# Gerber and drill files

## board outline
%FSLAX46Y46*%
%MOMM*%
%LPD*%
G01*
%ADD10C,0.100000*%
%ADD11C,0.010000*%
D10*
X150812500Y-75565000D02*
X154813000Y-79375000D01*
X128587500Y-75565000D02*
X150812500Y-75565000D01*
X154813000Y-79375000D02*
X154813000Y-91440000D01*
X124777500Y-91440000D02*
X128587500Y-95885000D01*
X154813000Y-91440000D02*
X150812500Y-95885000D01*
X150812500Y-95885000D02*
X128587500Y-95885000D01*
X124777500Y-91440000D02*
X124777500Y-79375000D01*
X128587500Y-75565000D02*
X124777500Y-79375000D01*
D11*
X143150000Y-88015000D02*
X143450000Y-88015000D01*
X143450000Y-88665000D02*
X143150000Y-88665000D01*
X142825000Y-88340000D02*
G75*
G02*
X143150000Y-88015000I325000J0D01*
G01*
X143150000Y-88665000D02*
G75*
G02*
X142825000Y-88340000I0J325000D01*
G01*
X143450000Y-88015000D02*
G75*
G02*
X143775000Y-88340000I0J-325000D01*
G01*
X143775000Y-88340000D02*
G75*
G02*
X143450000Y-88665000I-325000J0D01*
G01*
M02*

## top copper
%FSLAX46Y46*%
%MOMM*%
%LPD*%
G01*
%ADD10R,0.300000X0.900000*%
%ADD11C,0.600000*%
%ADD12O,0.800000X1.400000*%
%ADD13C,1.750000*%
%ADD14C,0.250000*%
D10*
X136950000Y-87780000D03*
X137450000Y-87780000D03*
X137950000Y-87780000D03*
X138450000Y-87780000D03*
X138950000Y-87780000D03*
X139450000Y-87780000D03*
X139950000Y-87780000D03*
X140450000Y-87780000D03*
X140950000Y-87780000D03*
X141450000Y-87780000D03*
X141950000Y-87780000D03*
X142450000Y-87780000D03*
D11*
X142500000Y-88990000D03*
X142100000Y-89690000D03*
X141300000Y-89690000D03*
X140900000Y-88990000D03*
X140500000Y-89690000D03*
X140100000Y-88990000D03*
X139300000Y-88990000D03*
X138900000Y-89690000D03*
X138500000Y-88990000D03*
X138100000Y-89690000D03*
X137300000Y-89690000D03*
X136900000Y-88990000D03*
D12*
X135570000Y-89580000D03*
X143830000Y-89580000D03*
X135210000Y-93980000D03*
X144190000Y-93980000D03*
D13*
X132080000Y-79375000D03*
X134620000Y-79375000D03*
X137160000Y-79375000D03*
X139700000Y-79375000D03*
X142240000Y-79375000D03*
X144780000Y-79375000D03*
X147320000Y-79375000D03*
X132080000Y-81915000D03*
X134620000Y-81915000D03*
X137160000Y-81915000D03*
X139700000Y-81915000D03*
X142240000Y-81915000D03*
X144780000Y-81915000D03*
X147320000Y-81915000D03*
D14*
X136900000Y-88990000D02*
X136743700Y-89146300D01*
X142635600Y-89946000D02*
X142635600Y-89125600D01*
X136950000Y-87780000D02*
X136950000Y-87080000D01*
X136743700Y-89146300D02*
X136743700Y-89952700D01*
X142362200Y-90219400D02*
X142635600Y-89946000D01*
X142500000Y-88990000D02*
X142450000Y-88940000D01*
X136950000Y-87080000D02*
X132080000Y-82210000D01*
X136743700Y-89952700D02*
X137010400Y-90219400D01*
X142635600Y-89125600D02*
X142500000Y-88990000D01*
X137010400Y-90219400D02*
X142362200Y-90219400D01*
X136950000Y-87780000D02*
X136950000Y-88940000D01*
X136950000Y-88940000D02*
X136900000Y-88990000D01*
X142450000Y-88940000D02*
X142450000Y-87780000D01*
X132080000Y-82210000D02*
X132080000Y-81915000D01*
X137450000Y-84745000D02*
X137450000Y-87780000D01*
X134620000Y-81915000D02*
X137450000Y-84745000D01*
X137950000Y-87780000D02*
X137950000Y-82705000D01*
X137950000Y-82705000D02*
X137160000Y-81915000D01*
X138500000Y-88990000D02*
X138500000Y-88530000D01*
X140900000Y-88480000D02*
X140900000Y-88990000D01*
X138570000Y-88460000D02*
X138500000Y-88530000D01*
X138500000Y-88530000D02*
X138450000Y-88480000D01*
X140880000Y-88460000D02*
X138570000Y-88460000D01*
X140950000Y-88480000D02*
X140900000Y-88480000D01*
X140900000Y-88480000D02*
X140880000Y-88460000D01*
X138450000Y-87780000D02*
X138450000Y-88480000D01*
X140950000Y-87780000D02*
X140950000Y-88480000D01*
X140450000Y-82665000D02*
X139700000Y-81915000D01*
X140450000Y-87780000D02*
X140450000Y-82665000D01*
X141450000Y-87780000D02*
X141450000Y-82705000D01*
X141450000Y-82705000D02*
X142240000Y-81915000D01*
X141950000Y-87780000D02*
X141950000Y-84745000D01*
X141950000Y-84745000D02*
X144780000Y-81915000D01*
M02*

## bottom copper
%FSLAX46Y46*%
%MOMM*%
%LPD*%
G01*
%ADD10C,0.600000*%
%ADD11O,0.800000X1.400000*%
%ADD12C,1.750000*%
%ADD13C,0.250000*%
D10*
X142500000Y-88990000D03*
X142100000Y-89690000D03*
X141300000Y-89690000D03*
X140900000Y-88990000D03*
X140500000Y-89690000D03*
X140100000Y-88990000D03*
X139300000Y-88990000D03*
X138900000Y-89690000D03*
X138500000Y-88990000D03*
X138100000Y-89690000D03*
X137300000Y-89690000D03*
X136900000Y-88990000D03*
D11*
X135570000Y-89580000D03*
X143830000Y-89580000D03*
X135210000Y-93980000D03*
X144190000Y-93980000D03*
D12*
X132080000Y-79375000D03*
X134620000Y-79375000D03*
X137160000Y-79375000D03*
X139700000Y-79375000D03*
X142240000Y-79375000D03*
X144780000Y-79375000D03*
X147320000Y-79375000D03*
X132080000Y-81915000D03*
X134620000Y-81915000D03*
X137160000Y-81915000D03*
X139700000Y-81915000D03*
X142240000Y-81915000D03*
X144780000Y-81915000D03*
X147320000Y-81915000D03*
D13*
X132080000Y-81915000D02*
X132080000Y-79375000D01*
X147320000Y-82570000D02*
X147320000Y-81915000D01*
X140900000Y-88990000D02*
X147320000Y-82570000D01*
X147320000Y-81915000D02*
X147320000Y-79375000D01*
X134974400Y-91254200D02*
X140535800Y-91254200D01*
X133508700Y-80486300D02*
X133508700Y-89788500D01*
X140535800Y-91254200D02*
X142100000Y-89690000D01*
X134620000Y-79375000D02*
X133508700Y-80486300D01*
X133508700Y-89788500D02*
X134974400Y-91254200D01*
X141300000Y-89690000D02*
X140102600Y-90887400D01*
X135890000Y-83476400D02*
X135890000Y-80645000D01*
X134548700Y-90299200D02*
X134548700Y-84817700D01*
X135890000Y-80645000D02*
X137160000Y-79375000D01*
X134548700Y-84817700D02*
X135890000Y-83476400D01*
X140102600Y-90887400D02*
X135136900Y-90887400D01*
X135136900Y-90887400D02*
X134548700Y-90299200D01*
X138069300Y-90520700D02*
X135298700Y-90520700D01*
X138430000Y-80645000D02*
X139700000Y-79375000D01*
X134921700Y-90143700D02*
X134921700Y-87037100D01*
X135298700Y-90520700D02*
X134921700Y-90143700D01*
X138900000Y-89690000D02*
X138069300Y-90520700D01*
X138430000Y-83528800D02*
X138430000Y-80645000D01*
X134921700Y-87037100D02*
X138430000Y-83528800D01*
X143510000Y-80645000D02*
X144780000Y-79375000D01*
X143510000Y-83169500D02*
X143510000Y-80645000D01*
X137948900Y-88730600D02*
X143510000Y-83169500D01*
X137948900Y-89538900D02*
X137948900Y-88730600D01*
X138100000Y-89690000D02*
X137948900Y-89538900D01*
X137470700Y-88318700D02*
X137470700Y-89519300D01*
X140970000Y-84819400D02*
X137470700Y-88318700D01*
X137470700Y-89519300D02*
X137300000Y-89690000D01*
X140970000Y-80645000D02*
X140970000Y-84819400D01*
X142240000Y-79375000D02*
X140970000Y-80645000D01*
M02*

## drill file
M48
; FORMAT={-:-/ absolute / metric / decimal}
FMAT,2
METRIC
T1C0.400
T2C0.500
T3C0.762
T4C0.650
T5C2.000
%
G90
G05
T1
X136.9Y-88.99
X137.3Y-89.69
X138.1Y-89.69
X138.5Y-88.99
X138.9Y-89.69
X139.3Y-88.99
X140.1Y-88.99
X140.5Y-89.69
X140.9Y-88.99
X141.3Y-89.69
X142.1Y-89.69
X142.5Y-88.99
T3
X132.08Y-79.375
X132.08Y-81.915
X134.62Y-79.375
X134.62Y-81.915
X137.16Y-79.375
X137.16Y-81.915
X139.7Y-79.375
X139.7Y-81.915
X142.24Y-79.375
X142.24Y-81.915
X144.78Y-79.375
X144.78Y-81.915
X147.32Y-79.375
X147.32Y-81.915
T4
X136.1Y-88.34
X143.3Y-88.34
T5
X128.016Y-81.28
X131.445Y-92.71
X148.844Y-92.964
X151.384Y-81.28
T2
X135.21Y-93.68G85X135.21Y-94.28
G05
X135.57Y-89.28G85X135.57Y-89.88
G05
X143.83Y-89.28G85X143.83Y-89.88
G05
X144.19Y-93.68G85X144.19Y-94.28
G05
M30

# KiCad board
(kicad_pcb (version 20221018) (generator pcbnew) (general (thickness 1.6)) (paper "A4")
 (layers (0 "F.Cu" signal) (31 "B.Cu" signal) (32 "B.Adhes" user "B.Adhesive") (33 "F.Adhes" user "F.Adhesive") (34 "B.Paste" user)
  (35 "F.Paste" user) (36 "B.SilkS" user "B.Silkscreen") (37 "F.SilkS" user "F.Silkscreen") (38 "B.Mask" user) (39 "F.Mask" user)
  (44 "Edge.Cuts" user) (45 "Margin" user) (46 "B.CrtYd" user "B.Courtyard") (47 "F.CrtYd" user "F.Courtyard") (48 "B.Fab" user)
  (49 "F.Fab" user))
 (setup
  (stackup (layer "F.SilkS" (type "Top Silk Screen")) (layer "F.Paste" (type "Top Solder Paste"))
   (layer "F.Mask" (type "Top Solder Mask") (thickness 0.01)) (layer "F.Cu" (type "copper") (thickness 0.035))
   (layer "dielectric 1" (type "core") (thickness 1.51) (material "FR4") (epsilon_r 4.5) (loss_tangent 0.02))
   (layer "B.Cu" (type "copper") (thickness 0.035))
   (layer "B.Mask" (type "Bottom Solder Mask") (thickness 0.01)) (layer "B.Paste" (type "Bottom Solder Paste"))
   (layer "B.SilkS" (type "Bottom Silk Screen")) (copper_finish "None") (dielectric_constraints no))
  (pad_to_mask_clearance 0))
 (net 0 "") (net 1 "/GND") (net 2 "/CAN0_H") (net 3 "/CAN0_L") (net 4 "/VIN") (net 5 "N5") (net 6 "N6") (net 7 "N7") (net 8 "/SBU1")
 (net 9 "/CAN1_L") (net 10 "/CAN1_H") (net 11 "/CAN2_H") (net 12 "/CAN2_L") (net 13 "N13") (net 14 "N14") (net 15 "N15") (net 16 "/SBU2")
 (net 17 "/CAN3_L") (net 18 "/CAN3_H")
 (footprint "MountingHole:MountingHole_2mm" (layer "F.Cu") (at 128.016 81.28)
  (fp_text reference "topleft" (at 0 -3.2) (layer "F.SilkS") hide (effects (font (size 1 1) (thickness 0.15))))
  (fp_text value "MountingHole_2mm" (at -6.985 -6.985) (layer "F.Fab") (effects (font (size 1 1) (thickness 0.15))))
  (pad "" np_thru_hole circle (at 0 0) (size 2 2) (drill 2) (layers "*.Cu" "*.Mask")))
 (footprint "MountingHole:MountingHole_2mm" (layer "F.Cu") (at 148.844 92.964)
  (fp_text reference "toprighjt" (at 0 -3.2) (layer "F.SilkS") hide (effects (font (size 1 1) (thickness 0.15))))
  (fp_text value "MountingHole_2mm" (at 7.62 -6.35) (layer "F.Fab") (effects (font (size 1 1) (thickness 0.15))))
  (pad "" np_thru_hole circle (at 0 0) (size 2 2) (drill 2) (layers "F&B.Cu" "*.Mask")))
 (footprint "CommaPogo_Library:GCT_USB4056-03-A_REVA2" (layer "F.Cu") (at 139.7 93.98)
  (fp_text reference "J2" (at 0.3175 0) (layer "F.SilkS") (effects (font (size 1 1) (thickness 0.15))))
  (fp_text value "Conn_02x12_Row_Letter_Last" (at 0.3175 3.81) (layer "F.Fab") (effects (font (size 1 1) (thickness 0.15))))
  (fp_line (start 3.45 -5.965) (end 3.75 -5.965) (stroke (width 0.01) (type solid)) (layer "Edge.Cuts"))
  (fp_line (start 3.75 -5.315) (end 3.45 -5.315) (stroke (width 0.01) (type solid)) (layer "Edge.Cuts"))
  (fp_arc (start 3.125 -5.64) (mid 3.22019 -5.86981) (end 3.45 -5.965) (stroke (width 0.01) (type solid)) (layer "Edge.Cuts"))
  (fp_arc (start 3.45 -5.315) (mid 3.22019 -5.41019) (end 3.125 -5.64) (stroke (width 0.01) (type solid)) (layer "Edge.Cuts"))
  (fp_arc (start 3.75 -5.965) (mid 3.97981 -5.86981) (end 4.075 -5.64) (stroke (width 0.01) (type solid)) (layer "Edge.Cuts"))
  (fp_arc (start 4.075 -5.64) (mid 3.97981 -5.41019) (end 3.75 -5.315) (stroke (width 0.01) (type solid)) (layer "Edge.Cuts"))
  (pad "" np_thru_hole circle (at -3.6 -5.64) (size 0.65 0.65) (drill 0.65) (layers "*.Cu" "*.Mask"))
  (pad "" np_thru_hole circle (at 3.6 -5.64) (size 0.65 0.65) (drill 0.65) (layers "*.Cu" "*.Mask"))
  (pad "A1" smd rect (at -2.75 -6.2) (size 0.3 0.9) (layers "F.Cu" "F.Paste" "F.Mask") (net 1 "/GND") (solder_mask_margin 0.102))
  (pad "A2" smd rect (at -2.25 -6.2) (size 0.3 0.9) (layers "F.Cu" "F.Paste" "F.Mask") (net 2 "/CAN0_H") (solder_mask_margin 0.102))
  (pad "A3" smd rect (at -1.75 -6.2) (size 0.3 0.9) (layers "F.Cu" "F.Paste" "F.Mask") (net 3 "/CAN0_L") (solder_mask_margin 0.102))
  (pad "A4" smd rect (at -1.25 -6.2) (size 0.3 0.9) (layers "F.Cu" "F.Paste" "F.Mask") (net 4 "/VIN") (solder_mask_margin 0.102))
  (pad "A5" smd rect (at -0.75 -6.2) (size 0.3 0.9) (layers "F.Cu" "F.Paste" "F.Mask") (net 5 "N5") (solder_mask_margin 0.102))
  (pad "A6" smd rect (at -0.25 -6.2) (size 0.3 0.9) (layers "F.Cu" "F.Paste" "F.Mask") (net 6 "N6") (solder_mask_margin 0.102))
  (pad "A7" smd rect (at 0.25 -6.2) (size 0.3 0.9) (layers "F.Cu" "F.Paste" "F.Mask") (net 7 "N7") (solder_mask_margin 0.102))
  (pad "A8" smd rect (at 0.75 -6.2) (size 0.3 0.9) (layers "F.Cu" "F.Paste" "F.Mask") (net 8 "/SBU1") (solder_mask_margin 0.102))
  (pad "A9" smd rect (at 1.25 -6.2) (size 0.3 0.9) (layers "F.Cu" "F.Paste" "F.Mask") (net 4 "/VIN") (solder_mask_margin 0.102))
  (pad "A10" smd rect (at 1.75 -6.2) (size 0.3 0.9) (layers "F.Cu" "F.Paste" "F.Mask") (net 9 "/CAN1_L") (solder_mask_margin 0.102))
  (pad "A11" smd rect (at 2.25 -6.2) (size 0.3 0.9) (layers "F.Cu" "F.Paste" "F.Mask") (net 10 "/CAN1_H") (solder_mask_margin 0.102))
  (pad "A12" smd rect (at 2.75 -6.2) (size 0.3 0.9) (layers "F.Cu" "F.Paste" "F.Mask") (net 1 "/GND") (solder_mask_margin 0.102))
  (pad "B1" thru_hole circle (at 2.8 -4.99) (size 0.6 0.6) (drill 0.4) (layers "*.Cu" "*.Mask") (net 1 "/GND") (solder_mask_margin 0.102))
  (pad "B2" thru_hole circle (at 2.4 -4.29) (size 0.6 0.6) (drill 0.4) (layers "*.Cu" "*.Mask") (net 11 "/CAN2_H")
   (solder_mask_margin 0.102))
  (pad "B3" thru_hole circle (at 1.6 -4.29) (size 0.6 0.6) (drill 0.4) (layers "*.Cu" "*.Mask") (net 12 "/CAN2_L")
   (solder_mask_margin 0.102))
  (pad "B4" thru_hole circle (at 1.2 -4.99) (size 0.6 0.6) (drill 0.4) (layers "*.Cu" "*.Mask") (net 4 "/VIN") (solder_mask_margin 0.102))
  (pad "B5" thru_hole circle (at 0.8 -4.29) (size 0.6 0.6) (drill 0.4) (layers "*.Cu" "*.Mask") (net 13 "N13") (solder_mask_margin 0.102))
  (pad "B6" thru_hole circle (at 0.4 -4.99) (size 0.6 0.6) (drill 0.4) (layers "*.Cu" "*.Mask") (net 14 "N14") (solder_mask_margin 0.102))
  (pad "B7" thru_hole circle (at -0.4 -4.99) (size 0.6 0.6) (drill 0.4) (layers "*.Cu" "*.Mask") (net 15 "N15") (solder_mask_margin 0.102))
  (pad "B8" thru_hole circle (at -0.8 -4.29) (size 0.6 0.6) (drill 0.4) (layers "*.Cu" "*.Mask") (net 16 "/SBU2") (solder_mask_margin 0.102))
  (pad "B9" thru_hole circle (at -1.2 -4.99) (size 0.6 0.6) (drill 0.4) (layers "*.Cu" "*.Mask") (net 4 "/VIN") (solder_mask_margin 0.102))
  (pad "B10" thru_hole circle (at -1.6 -4.29) (size 0.6 0.6) (drill 0.4) (layers "*.Cu" "*.Mask") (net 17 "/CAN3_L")
   (solder_mask_margin 0.102))
  (pad "B11" thru_hole circle (at -2.4 -4.29) (size 0.6 0.6) (drill 0.4) (layers "*.Cu" "*.Mask") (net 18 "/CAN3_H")
   (solder_mask_margin 0.102))
  (pad "B12" thru_hole circle (at -2.8 -4.99) (size 0.6 0.6) (drill 0.4) (layers "*.Cu" "*.Mask") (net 1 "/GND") (solder_mask_margin 0.102))
  (pad "S1" thru_hole oval (at -4.13 -4.4) (size 0.8 1.4) (drill oval 0.5 1.1) (layers "*.Cu" "*.Mask") (solder_mask_margin 0.102))
  (pad "S2" thru_hole oval (at 4.13 -4.4) (size 0.8 1.4) (drill oval 0.5 1.1) (layers "*.Cu" "*.Mask") (solder_mask_margin 0.102))
  (pad "S3" thru_hole oval (at -4.49 0) (size 0.8 1.4) (drill oval 0.5 1.1) (layers "*.Cu" "*.Mask") (solder_mask_margin 0.102))
  (pad "S4" thru_hole oval (at 4.49 0) (size 0.8 1.4) (drill oval 0.5 1.1) (layers "*.Cu" "*.Mask") (solder_mask_margin 0.102)))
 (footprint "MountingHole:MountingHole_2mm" (layer "F.Cu") (at 151.384 81.28)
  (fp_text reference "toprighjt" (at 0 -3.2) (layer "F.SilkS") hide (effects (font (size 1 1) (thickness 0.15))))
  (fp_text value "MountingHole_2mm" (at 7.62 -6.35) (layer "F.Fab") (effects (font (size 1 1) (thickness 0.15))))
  (pad "" np_thru_hole circle (at 0 0) (size 2 2) (drill 2) (layers "*.Cu" "*.Mask")))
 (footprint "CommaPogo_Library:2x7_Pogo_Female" (layer "F.Cu") (at 139.7 83.82)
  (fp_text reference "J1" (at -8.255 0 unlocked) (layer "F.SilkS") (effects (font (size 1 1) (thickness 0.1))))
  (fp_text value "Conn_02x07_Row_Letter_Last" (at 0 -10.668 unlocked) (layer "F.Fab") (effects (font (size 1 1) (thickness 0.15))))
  (pad "1" thru_hole circle (at -7.62 -4.445) (size 1.75 1.75) (drill 0.762) (layers "*.Cu" "*.Mask") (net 1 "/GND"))
  (pad "2" thru_hole circle (at -5.08 -4.445) (size 1.75 1.75) (drill 0.762) (layers "*.Cu" "*.Mask") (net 11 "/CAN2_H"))
  (pad "3" thru_hole circle (at -2.54 -4.445) (size 1.75 1.75) (drill 0.762) (layers "*.Cu" "*.Mask") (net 12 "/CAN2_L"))
  (pad "4" thru_hole circle (at 0 -4.445) (size 1.75 1.75) (drill 0.762) (layers "*.Cu" "*.Mask") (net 16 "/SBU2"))
  (pad "5" thru_hole circle (at 2.54 -4.445) (size 1.75 1.75) (drill 0.762) (layers "*.Cu" "*.Mask") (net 18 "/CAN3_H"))
  (pad "6" thru_hole circle (at 5.08 -4.445) (size 1.75 1.75) (drill 0.762) (layers "*.Cu" "*.Mask") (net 17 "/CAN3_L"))
  (pad "7" thru_hole circle (at 7.62 -4.445) (size 1.75 1.75) (drill 0.762) (layers "*.Cu" "*.Mask") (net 4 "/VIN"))
  (pad "8" thru_hole circle (at -7.62 -1.905) (size 1.75 1.75) (drill 0.762) (layers "*.Cu" "*.Mask") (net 1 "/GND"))
  (pad "9" thru_hole circle (at -5.08 -1.905) (size 1.75 1.75) (drill 0.762) (layers "*.Cu" "*.Mask") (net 2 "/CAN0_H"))
  (pad "10" thru_hole circle (at -2.54 -1.905) (size 1.75 1.75) (drill 0.762) (layers "*.Cu" "*.Mask") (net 3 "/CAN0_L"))
  (pad "11" thru_hole circle (at 0 -1.905) (size 1.75 1.75) (drill 0.762) (layers "*.Cu" "*.Mask") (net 8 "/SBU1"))
  (pad "12" thru_hole circle (at 2.54 -1.905) (size 1.75 1.75) (drill 0.762) (layers "*.Cu" "*.Mask") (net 9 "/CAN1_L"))
  (pad "13" thru_hole circle (at 5.08 -1.905) (size 1.75 1.75) (drill 0.762) (layers "*.Cu" "*.Mask") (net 10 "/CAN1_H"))
  (pad "14" thru_hole circle (at 7.62 -1.905) (size 1.75 1.75) (drill 0.762) (layers "*.Cu" "*.Mask") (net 4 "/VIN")))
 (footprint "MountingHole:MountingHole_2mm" (layer "F.Cu") (at 131.445 92.71)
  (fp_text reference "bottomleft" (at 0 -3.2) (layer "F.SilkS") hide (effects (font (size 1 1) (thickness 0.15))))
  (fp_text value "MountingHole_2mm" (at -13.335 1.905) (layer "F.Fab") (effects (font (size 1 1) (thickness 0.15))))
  (pad "" np_thru_hole circle (at 0 0) (size 2 2) (drill 2) (layers "F&B.Cu" "*.Mask")))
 (gr_line (start 150.8125 75.565) (end 154.813 79.375) (stroke (width 0.1) (type default)) (layer "Edge.Cuts"))
 (gr_line (start 128.5875 75.565) (end 150.8125 75.565) (stroke (width 0.1) (type default)) (layer "Edge.Cuts"))
 (gr_line (start 154.813 79.375) (end 154.813 91.44) (stroke (width 0.1) (type default)) (layer "Edge.Cuts"))
 (gr_line (start 124.7775 91.44) (end 128.5875 95.885) (stroke (width 0.1) (type default)) (layer "Edge.Cuts"))
 (gr_line (start 154.813 91.44) (end 150.8125 95.885) (stroke (width 0.1) (type default)) (layer "Edge.Cuts"))
 (gr_line (start 150.8125 95.885) (end 128.5875 95.885) (stroke (width 0.1) (type default)) (layer "Edge.Cuts"))
 (gr_line (start 124.7775 91.44) (end 124.7775 79.375) (stroke (width 0.1) (type default)) (layer "Edge.Cuts"))
 (gr_line (start 128.5875 75.565) (end 124.7775 79.375) (stroke (width 0.1) (type default)) (layer "Edge.Cuts"))
 (segment (start 136.9 88.99) (end 136.7437 89.1463) (width 0.25) (layer "F.Cu") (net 1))
 (segment (start 142.6356 89.946) (end 142.6356 89.1256) (width 0.25) (layer "F.Cu") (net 1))
 (segment (start 136.95 87.78) (end 136.95 87.08) (width 0.25) (layer "F.Cu") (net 1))
 (segment (start 136.7437 89.1463) (end 136.7437 89.9527) (width 0.25) (layer "F.Cu") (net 1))
 (segment (start 142.3622 90.2194) (end 142.6356 89.946) (width 0.25) (layer "F.Cu") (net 1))
 (segment (start 142.5 88.99) (end 142.45 88.94) (width 0.25) (layer "F.Cu") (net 1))
 (segment (start 136.95 87.08) (end 132.08 82.21) (width 0.25) (layer "F.Cu") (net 1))
 (segment (start 136.7437 89.9527) (end 137.0104 90.2194) (width 0.25) (layer "F.Cu") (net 1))
 (segment (start 142.6356 89.1256) (end 142.5 88.99) (width 0.25) (layer "F.Cu") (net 1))
 (segment (start 137.0104 90.2194) (end 142.3622 90.2194) (width 0.25) (layer "F.Cu") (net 1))
 (segment (start 136.95 87.78) (end 136.95 88.94) (width 0.25) (layer "F.Cu") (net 1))
 (segment (start 136.95 88.94) (end 136.9 88.99) (width 0.25) (layer "F.Cu") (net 1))
 (segment (start 142.45 88.94) (end 142.45 87.78) (width 0.25) (layer "F.Cu") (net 1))
 (segment (start 132.08 82.21) (end 132.08 81.915) (width 0.25) (layer "F.Cu") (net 1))
 (segment (start 132.08 81.915) (end 132.08 79.375) (width 0.25) (layer "B.Cu") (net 1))
 (segment (start 137.45 84.745) (end 137.45 87.78) (width 0.25) (layer "F.Cu") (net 2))
 (segment (start 134.62 81.915) (end 137.45 84.745) (width 0.25) (layer "F.Cu") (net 2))
 (segment (start 137.95 87.78) (end 137.95 82.705) (width 0.25) (layer "F.Cu") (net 3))
 (segment (start 137.95 82.705) (end 137.16 81.915) (width 0.25) (layer "F.Cu") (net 3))
 (segment (start 138.5 88.99) (end 138.5 88.53) (width 0.25) (layer "F.Cu") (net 4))
 (segment (start 140.9 88.48) (end 140.9 88.99) (width 0.25) (layer "F.Cu") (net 4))
 (segment (start 138.57 88.46) (end 138.5 88.53) (width 0.25) (layer "F.Cu") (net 4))
 (segment (start 138.5 88.53) (end 138.45 88.48) (width 0.25) (layer "F.Cu") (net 4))
 (segment (start 140.88 88.46) (end 138.57 88.46) (width 0.25) (layer "F.Cu") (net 4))
 (segment (start 140.95 88.48) (end 140.9 88.48) (width 0.25) (layer "F.Cu") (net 4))
 (segment (start 140.9 88.48) (end 140.88 88.46) (width 0.25) (layer "F.Cu") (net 4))
 (segment (start 138.45 87.78) (end 138.45 88.48) (width 0.25) (layer "F.Cu") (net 4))
 (segment (start 140.95 87.78) (end 140.95 88.48) (width 0.25) (layer "F.Cu") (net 4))
 (segment (start 147.32 82.57) (end 147.32 81.915) (width 0.25) (layer "B.Cu") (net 4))
 (segment (start 140.9 88.99) (end 147.32 82.57) (width 0.25) (layer "B.Cu") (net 4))
 (segment (start 147.32 81.915) (end 147.32 79.375) (width 0.25) (layer "B.Cu") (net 4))
 (segment (start 140.45 82.665) (end 139.7 81.915) (width 0.25) (layer "F.Cu") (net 8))
 (segment (start 140.45 87.78) (end 140.45 82.665) (width 0.25) (layer "F.Cu") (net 8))
 (segment (start 141.45 87.78) (end 141.45 82.705) (width 0.25) (layer "F.Cu") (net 9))
 (segment (start 141.45 82.705) (end 142.24 81.915) (width 0.25) (layer "F.Cu") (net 9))
 (segment (start 141.95 87.78) (end 141.95 84.745) (width 0.25) (layer "F.Cu") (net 10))
 (segment (start 141.95 84.745) (end 144.78 81.915) (width 0.25) (layer "F.Cu") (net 10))
 (segment (start 134.9744 91.2542) (end 140.5358 91.2542) (width 0.25) (layer "B.Cu") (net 11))
 (segment (start 133.5087 80.4863) (end 133.5087 89.7885) (width 0.25) (layer "B.Cu") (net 11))
 (segment (start 140.5358 91.2542) (end 142.1 89.69) (width 0.25) (layer "B.Cu") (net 11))
 (segment (start 134.62 79.375) (end 133.5087 80.4863) (width 0.25) (layer "B.Cu") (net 11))
 (segment (start 133.5087 89.7885) (end 134.9744 91.2542) (width 0.25) (layer "B.Cu") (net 11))
 (segment (start 141.3 89.69) (end 140.1026 90.8874) (width 0.25) (layer "B.Cu") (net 12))
 (segment (start 135.89 83.4764) (end 135.89 80.645) (width 0.25) (layer "B.Cu") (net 12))
 (segment (start 134.5487 90.2992) (end 134.5487 84.8177) (width 0.25) (layer "B.Cu") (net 12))
 (segment (start 135.89 80.645) (end 137.16 79.375) (width 0.25) (layer "B.Cu") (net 12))
 (segment (start 134.5487 84.8177) (end 135.89 83.4764) (width 0.25) (layer "B.Cu") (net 12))
 (segment (start 140.1026 90.8874) (end 135.1369 90.8874) (width 0.25) (layer "B.Cu") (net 12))
 (segment (start 135.1369 90.8874) (end 134.5487 90.2992) (width 0.25) (layer "B.Cu") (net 12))
 (segment (start 138.0693 90.5207) (end 135.2987 90.5207) (width 0.25) (layer "B.Cu") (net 16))
 (segment (start 138.43 80.645) (end 139.7 79.375) (width 0.25) (layer "B.Cu") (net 16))
 (segment (start 134.9217 90.1437) (end 134.9217 87.0371) (width 0.25) (layer "B.Cu") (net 16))
 (segment (start 135.2987 90.5207) (end 134.9217 90.1437) (width 0.25) (layer "B.Cu") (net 16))
 (segment (start 138.9 89.69) (end 138.0693 90.5207) (width 0.25) (layer "B.Cu") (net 16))
 (segment (start 138.43 83.5288) (end 138.43 80.645) (width 0.25) (layer "B.Cu") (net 16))
 (segment (start 134.9217 87.0371) (end 138.43 83.5288) (width 0.25) (layer "B.Cu") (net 16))
 (segment (start 143.51 80.645) (end 144.78 79.375) (width 0.25) (layer "B.Cu") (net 17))
 (segment (start 143.51 83.1695) (end 143.51 80.645) (width 0.25) (layer "B.Cu") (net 17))
 (segment (start 137.9489 88.7306) (end 143.51 83.1695) (width 0.25) (layer "B.Cu") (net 17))
 (segment (start 137.9489 89.5389) (end 137.9489 88.7306) (width 0.25) (layer "B.Cu") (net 17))
 (segment (start 138.1 89.69) (end 137.9489 89.5389) (width 0.25) (layer "B.Cu") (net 17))
 (segment (start 137.4707 88.3187) (end 137.4707 89.5193) (width 0.25) (layer "B.Cu") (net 18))
 (segment (start 140.97 84.8194) (end 137.4707 88.3187) (width 0.25) (layer "B.Cu") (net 18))
 (segment (start 137.4707 89.5193) (end 137.3 89.69) (width 0.25) (layer "B.Cu") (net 18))
 (segment (start 140.97 80.645) (end 140.97 84.8194) (width 0.25) (layer "B.Cu") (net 18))
 (segment (start 142.24 79.375) (end 140.97 80.645) (width 0.25) (layer "B.Cu") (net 18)))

